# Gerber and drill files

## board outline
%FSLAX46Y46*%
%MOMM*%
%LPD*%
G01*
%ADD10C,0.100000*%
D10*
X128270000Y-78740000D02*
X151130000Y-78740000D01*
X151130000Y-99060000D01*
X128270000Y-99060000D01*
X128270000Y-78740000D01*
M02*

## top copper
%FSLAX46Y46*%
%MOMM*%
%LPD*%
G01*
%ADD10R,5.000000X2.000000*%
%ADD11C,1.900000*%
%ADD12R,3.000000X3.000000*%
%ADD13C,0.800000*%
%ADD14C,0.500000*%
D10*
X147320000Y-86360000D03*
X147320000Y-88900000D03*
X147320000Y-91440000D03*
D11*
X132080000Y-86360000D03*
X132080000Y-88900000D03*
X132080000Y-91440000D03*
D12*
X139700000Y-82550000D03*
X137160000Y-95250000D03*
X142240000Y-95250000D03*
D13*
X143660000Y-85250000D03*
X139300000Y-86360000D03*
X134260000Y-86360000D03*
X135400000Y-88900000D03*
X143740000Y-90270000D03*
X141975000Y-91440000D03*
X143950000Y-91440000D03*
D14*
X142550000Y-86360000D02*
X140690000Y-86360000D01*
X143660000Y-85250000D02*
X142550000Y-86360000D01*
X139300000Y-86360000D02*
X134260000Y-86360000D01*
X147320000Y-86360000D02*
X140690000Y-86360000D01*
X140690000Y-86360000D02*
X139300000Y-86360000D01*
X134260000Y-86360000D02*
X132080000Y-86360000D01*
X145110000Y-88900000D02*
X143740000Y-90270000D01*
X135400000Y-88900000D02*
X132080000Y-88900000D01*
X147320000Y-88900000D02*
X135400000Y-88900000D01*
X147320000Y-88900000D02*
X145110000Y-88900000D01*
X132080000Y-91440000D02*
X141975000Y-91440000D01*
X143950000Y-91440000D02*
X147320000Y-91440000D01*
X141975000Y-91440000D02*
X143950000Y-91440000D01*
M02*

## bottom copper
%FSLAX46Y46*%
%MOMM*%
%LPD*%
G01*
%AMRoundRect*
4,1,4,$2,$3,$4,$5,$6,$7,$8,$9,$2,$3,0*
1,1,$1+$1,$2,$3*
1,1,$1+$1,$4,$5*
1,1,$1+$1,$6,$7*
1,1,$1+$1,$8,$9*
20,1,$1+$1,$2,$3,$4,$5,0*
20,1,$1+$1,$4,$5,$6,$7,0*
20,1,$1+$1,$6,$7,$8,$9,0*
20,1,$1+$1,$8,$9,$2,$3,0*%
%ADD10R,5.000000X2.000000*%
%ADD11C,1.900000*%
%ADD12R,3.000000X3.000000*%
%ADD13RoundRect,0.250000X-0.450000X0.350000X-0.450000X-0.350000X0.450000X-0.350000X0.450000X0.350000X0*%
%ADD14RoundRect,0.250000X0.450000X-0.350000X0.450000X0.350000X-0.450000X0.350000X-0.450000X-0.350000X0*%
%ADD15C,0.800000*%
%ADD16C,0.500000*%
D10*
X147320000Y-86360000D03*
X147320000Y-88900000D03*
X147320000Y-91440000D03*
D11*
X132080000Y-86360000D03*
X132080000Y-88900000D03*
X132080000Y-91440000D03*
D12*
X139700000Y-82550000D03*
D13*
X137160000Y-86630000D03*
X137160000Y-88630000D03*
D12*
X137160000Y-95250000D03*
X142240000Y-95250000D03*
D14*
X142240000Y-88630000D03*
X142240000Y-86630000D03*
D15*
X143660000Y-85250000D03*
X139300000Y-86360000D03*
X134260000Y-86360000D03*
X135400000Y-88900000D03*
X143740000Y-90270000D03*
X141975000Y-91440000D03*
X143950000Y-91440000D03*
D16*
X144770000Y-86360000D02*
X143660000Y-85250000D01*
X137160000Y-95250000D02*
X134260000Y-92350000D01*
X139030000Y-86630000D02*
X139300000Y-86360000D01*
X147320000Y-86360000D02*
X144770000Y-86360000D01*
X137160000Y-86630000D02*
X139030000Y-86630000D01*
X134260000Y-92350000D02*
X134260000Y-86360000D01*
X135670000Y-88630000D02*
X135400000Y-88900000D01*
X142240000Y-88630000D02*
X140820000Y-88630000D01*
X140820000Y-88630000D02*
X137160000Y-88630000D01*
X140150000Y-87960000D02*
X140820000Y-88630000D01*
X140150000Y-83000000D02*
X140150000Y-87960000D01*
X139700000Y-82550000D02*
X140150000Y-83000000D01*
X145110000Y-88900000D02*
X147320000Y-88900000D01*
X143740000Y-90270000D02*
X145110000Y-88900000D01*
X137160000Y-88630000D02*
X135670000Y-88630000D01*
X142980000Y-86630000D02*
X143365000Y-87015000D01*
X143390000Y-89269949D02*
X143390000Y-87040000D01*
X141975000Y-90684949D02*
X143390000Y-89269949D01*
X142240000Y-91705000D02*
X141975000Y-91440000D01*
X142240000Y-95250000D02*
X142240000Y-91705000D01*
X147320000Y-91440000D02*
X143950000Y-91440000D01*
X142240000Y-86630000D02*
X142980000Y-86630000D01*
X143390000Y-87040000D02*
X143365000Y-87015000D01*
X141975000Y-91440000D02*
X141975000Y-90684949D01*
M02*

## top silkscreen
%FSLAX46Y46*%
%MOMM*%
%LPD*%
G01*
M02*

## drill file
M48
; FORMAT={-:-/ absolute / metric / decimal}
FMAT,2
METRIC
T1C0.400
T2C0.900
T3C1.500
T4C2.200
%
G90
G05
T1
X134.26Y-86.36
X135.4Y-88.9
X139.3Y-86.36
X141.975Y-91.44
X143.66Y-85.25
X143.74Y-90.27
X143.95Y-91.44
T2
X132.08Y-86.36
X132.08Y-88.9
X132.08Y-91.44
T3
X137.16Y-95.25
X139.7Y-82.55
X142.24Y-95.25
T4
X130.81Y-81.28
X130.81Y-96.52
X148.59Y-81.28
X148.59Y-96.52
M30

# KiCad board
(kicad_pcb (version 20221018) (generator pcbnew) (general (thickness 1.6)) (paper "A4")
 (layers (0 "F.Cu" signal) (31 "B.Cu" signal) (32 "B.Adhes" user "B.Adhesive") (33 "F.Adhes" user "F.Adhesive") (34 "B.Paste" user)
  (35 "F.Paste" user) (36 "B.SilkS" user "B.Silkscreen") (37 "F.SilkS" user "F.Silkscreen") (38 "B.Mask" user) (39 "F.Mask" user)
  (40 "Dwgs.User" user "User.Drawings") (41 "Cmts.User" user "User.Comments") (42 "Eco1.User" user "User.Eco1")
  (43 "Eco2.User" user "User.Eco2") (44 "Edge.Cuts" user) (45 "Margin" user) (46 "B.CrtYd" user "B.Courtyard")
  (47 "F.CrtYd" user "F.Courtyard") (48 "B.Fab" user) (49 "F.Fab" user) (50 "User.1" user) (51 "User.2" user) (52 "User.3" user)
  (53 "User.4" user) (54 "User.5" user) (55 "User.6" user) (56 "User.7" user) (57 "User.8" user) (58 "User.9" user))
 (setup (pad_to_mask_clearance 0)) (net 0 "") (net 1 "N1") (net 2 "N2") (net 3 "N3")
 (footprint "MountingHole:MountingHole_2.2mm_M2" (layer "F.Cu") (at 130.81 81.28)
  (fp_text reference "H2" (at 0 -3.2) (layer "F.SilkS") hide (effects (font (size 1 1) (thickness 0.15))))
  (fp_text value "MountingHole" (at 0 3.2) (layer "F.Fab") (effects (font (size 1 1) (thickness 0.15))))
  (pad "" np_thru_hole circle (at 0 0) (size 2.2 2.2) (drill 2.2) (layers "*.Cu" "*.Mask")))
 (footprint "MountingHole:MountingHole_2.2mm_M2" (layer "F.Cu") (at 130.81 96.52)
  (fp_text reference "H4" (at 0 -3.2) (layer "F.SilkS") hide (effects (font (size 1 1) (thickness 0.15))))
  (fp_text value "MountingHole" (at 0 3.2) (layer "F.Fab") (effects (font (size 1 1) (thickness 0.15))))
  (pad "" np_thru_hole circle (at 0 0) (size 2.2 2.2) (drill 2.2) (layers "*.Cu" "*.Mask")))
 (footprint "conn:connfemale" (layer "F.Cu") (at 147.32 88.9)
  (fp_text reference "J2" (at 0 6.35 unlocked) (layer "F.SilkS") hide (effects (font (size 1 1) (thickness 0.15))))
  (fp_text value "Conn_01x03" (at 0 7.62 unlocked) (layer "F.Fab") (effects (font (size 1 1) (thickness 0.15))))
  (pad "1" smd rect (at 0 -2.54) (size 5 2) (layers "F.Cu" "F.Paste" "F.Mask") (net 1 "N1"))
  (pad "1" smd rect (at 0 -2.54) (size 5 2) (layers "B.Cu" "B.Paste" "B.Mask") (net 1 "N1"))
  (pad "2" smd rect (at 0 0) (size 5 2) (layers "F.Cu" "F.Paste" "F.Mask") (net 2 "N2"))
  (pad "2" smd rect (at 0 0) (size 5 2) (layers "B.Cu" "B.Paste" "B.Mask") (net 2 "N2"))
  (pad "3" smd rect (at 0 2.54) (size 5 2) (layers "F.Cu" "F.Paste" "F.Mask") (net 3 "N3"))
  (pad "3" smd rect (at 0 2.54) (size 5 2) (layers "B.Cu" "B.Paste" "B.Mask") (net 3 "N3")))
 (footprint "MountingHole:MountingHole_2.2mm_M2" (layer "F.Cu") (at 148.59 96.52)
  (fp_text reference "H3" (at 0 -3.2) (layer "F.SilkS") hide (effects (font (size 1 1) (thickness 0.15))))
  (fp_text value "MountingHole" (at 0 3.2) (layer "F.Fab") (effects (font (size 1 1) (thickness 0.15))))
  (pad "" np_thru_hole circle (at 0 0) (size 2.2 2.2) (drill 2.2) (layers "*.Cu" "*.Mask")))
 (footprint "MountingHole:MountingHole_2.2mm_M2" (layer "F.Cu") (at 148.59 81.28)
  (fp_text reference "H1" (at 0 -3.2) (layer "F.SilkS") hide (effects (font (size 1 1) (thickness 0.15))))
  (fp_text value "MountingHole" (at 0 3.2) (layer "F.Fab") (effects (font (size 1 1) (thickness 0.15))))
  (pad "" np_thru_hole circle (at 0 0) (size 2.2 2.2) (drill 2.2) (layers "*.Cu" "*.Mask")))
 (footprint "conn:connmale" (layer "F.Cu") (at 132.08 88.9)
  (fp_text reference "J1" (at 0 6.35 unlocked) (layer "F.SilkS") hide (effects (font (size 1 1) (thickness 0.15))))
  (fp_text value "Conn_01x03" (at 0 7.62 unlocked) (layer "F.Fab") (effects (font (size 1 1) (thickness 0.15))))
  (pad "1" thru_hole circle (at 0 -2.54) (size 1.9 1.9) (drill 0.9) (layers "*.Cu" "*.Mask") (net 1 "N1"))
  (pad "2" thru_hole circle (at 0 0) (size 1.9 1.9) (drill 0.9) (layers "*.Cu" "*.Mask") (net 2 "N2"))
  (pad "3" thru_hole circle (at 0 2.54) (size 1.9 1.9) (drill 0.9) (layers "*.Cu" "*.Mask") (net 3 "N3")))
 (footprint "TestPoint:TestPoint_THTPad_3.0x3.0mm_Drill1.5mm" (layer "B.Cu") (at 139.7 82.55 -90)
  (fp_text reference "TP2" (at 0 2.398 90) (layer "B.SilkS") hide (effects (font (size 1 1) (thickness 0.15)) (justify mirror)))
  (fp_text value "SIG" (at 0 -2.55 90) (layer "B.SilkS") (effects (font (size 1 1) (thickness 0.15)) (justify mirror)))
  (pad "1" thru_hole rect (at 0 0 270) (size 3 3) (drill 1.5) (layers "*.Cu" "*.Mask") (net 2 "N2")))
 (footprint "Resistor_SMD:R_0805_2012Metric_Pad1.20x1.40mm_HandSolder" (layer "B.Cu") (at 137.16 87.63 -90)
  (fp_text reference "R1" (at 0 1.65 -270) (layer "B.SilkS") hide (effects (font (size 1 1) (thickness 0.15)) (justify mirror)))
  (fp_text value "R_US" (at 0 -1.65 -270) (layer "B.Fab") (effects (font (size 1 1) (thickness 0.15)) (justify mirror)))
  (pad "1" smd roundrect (at -1 0 270) (size 1.2 1.4) (layers "B.Cu" "B.Paste" "B.Mask") (roundrect_rratio 0.2083333333) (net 1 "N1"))
  (pad "2" smd roundrect (at 1 0 270) (size 1.2 1.4) (layers "B.Cu" "B.Paste" "B.Mask") (roundrect_rratio 0.2083333333) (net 2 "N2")))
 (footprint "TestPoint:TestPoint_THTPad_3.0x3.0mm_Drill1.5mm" (layer "B.Cu") (at 137.16 95.25 180)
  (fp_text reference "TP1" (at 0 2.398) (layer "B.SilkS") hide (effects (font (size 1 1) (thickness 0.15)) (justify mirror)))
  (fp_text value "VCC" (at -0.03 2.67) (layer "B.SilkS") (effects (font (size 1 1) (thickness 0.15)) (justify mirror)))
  (pad "1" thru_hole rect (at 0 0 180) (size 3 3) (drill 1.5) (layers "*.Cu" "*.Mask") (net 1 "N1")))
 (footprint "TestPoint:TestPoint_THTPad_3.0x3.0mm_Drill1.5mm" (layer "B.Cu") (at 142.24 95.25 180)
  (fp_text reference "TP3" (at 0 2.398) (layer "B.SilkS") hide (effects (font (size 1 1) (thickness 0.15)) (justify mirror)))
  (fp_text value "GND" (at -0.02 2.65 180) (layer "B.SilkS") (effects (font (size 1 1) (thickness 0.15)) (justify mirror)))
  (pad "1" thru_hole rect (at 0 0 180) (size 3 3) (drill 1.5) (layers "*.Cu" "*.Mask") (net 3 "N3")))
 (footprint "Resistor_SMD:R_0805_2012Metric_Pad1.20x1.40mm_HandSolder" (layer "B.Cu") (at 142.24 87.63 90)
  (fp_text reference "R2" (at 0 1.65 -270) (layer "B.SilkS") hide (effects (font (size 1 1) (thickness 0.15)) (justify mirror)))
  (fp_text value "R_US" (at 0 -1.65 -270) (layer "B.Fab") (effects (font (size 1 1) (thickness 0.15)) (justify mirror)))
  (pad "1" smd roundrect (at -1 0 90) (size 1.2 1.4) (layers "B.Cu" "B.Paste" "B.Mask") (roundrect_rratio 0.2083333333) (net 2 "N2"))
  (pad "2" smd roundrect (at 1 0 90) (size 1.2 1.4) (layers "B.Cu" "B.Paste" "B.Mask") (roundrect_rratio 0.2083333333) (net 3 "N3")))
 (gr_rect (start 128.27 78.74) (end 151.13 99.06) (stroke (width 0.1) (type default)) (fill none) (layer "Edge.Cuts"))
 (segment (start 142.55 86.36) (end 140.69 86.36) (width 0.5) (layer "F.Cu") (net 1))
 (segment (start 143.66 85.25) (end 142.55 86.36) (width 0.5) (layer "F.Cu") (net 1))
 (segment (start 139.3 86.36) (end 134.26 86.36) (width 0.5) (layer "F.Cu") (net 1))
 (segment (start 147.32 86.36) (end 140.69 86.36) (width 0.5) (layer "F.Cu") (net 1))
 (segment (start 140.69 86.36) (end 139.3 86.36) (width 0.5) (layer "F.Cu") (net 1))
 (segment (start 134.26 86.36) (end 132.08 86.36) (width 0.5) (layer "F.Cu") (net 1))
 (via (at 143.66 85.25) (size 0.8) (drill 0.4) (layers "F.Cu" "B.Cu") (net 1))
 (via (at 139.3 86.36) (size 0.8) (drill 0.4) (layers "F.Cu" "B.Cu") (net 1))
 (via (at 134.26 86.36) (size 0.8) (drill 0.4) (layers "F.Cu" "B.Cu") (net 1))
 (segment (start 144.77 86.36) (end 143.66 85.25) (width 0.5) (layer "B.Cu") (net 1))
 (segment (start 137.16 95.25) (end 134.26 92.35) (width 0.5) (layer "B.Cu") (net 1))
 (segment (start 139.03 86.63) (end 139.3 86.36) (width 0.5) (layer "B.Cu") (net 1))
 (segment (start 147.32 86.36) (end 144.77 86.36) (width 0.5) (layer "B.Cu") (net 1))
 (segment (start 137.16 86.63) (end 139.03 86.63) (width 0.5) (layer "B.Cu") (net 1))
 (segment (start 134.26 92.35) (end 134.26 86.36) (width 0.5) (layer "B.Cu") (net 1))
 (segment (start 145.11 88.9) (end 143.74 90.27) (width 0.5) (layer "F.Cu") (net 2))
 (segment (start 135.4 88.9) (end 132.08 88.9) (width 0.5) (layer "F.Cu") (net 2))
 (segment (start 147.32 88.9) (end 135.4 88.9) (width 0.5) (layer "F.Cu") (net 2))
 (segment (start 147.32 88.9) (end 145.11 88.9) (width 0.5) (layer "F.Cu") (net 2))
 (via (at 135.4 88.9) (size 0.8) (drill 0.4) (layers "F.Cu" "B.Cu") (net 2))
 (via (at 143.74 90.27) (size 0.8) (drill 0.4) (layers "F.Cu" "B.Cu") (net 2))
 (segment (start 135.67 88.63) (end 135.4 88.9) (width 0.5) (layer "B.Cu") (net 2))
 (segment (start 142.24 88.63) (end 140.82 88.63) (width 0.5) (layer "B.Cu") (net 2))
 (segment (start 140.82 88.63) (end 137.16 88.63) (width 0.5) (layer "B.Cu") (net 2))
 (segment (start 140.15 87.96) (end 140.82 88.63) (width 0.5) (layer "B.Cu") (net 2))
 (segment (start 140.15 83) (end 140.15 87.96) (width 0.5) (layer "B.Cu") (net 2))
 (segment (start 139.7 82.55) (end 140.15 83) (width 0.5) (layer "B.Cu") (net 2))
 (segment (start 145.11 88.9) (end 147.32 88.9) (width 0.5) (layer "B.Cu") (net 2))
 (segment (start 143.74 90.27) (end 145.11 88.9) (width 0.5) (layer "B.Cu") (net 2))
 (segment (start 137.16 88.63) (end 135.67 88.63) (width 0.5) (layer "B.Cu") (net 2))
 (segment (start 132.08 91.44) (end 141.975 91.44) (width 0.5) (layer "F.Cu") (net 3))
 (segment (start 143.95 91.44) (end 147.32 91.44) (width 0.5) (layer "F.Cu") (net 3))
 (segment (start 141.975 91.44) (end 143.95 91.44) (width 0.5) (layer "F.Cu") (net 3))
 (via (at 141.975 91.44) (size 0.8) (drill 0.4) (layers "F.Cu" "B.Cu") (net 3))
 (via (at 143.95 91.44) (size 0.8) (drill 0.4) (layers "F.Cu" "B.Cu") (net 3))
 (segment (start 142.98 86.63) (end 143.365 87.015) (width 0.5) (layer "B.Cu") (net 3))
 (segment (start 143.39 89.269949) (end 143.39 87.04) (width 0.5) (layer "B.Cu") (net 3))
 (segment (start 141.975 90.684949) (end 143.39 89.269949) (width 0.5) (layer "B.Cu") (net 3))
 (segment (start 142.24 91.705) (end 141.975 91.44) (width 0.5) (layer "B.Cu") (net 3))
 (segment (start 142.24 95.25) (end 142.24 91.705) (width 0.5) (layer "B.Cu") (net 3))
 (segment (start 147.32 91.44) (end 143.95 91.44) (width 0.5) (layer "B.Cu") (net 3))
 (segment (start 142.24 86.63) (end 142.98 86.63) (width 0.5) (layer "B.Cu") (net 3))
 (segment (start 143.39 87.04) (end 143.365 87.015) (width 0.5) (layer "B.Cu") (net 3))
 (segment (start 141.975 91.44) (end 141.975 90.684949) (width 0.5) (layer "B.Cu") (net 3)))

